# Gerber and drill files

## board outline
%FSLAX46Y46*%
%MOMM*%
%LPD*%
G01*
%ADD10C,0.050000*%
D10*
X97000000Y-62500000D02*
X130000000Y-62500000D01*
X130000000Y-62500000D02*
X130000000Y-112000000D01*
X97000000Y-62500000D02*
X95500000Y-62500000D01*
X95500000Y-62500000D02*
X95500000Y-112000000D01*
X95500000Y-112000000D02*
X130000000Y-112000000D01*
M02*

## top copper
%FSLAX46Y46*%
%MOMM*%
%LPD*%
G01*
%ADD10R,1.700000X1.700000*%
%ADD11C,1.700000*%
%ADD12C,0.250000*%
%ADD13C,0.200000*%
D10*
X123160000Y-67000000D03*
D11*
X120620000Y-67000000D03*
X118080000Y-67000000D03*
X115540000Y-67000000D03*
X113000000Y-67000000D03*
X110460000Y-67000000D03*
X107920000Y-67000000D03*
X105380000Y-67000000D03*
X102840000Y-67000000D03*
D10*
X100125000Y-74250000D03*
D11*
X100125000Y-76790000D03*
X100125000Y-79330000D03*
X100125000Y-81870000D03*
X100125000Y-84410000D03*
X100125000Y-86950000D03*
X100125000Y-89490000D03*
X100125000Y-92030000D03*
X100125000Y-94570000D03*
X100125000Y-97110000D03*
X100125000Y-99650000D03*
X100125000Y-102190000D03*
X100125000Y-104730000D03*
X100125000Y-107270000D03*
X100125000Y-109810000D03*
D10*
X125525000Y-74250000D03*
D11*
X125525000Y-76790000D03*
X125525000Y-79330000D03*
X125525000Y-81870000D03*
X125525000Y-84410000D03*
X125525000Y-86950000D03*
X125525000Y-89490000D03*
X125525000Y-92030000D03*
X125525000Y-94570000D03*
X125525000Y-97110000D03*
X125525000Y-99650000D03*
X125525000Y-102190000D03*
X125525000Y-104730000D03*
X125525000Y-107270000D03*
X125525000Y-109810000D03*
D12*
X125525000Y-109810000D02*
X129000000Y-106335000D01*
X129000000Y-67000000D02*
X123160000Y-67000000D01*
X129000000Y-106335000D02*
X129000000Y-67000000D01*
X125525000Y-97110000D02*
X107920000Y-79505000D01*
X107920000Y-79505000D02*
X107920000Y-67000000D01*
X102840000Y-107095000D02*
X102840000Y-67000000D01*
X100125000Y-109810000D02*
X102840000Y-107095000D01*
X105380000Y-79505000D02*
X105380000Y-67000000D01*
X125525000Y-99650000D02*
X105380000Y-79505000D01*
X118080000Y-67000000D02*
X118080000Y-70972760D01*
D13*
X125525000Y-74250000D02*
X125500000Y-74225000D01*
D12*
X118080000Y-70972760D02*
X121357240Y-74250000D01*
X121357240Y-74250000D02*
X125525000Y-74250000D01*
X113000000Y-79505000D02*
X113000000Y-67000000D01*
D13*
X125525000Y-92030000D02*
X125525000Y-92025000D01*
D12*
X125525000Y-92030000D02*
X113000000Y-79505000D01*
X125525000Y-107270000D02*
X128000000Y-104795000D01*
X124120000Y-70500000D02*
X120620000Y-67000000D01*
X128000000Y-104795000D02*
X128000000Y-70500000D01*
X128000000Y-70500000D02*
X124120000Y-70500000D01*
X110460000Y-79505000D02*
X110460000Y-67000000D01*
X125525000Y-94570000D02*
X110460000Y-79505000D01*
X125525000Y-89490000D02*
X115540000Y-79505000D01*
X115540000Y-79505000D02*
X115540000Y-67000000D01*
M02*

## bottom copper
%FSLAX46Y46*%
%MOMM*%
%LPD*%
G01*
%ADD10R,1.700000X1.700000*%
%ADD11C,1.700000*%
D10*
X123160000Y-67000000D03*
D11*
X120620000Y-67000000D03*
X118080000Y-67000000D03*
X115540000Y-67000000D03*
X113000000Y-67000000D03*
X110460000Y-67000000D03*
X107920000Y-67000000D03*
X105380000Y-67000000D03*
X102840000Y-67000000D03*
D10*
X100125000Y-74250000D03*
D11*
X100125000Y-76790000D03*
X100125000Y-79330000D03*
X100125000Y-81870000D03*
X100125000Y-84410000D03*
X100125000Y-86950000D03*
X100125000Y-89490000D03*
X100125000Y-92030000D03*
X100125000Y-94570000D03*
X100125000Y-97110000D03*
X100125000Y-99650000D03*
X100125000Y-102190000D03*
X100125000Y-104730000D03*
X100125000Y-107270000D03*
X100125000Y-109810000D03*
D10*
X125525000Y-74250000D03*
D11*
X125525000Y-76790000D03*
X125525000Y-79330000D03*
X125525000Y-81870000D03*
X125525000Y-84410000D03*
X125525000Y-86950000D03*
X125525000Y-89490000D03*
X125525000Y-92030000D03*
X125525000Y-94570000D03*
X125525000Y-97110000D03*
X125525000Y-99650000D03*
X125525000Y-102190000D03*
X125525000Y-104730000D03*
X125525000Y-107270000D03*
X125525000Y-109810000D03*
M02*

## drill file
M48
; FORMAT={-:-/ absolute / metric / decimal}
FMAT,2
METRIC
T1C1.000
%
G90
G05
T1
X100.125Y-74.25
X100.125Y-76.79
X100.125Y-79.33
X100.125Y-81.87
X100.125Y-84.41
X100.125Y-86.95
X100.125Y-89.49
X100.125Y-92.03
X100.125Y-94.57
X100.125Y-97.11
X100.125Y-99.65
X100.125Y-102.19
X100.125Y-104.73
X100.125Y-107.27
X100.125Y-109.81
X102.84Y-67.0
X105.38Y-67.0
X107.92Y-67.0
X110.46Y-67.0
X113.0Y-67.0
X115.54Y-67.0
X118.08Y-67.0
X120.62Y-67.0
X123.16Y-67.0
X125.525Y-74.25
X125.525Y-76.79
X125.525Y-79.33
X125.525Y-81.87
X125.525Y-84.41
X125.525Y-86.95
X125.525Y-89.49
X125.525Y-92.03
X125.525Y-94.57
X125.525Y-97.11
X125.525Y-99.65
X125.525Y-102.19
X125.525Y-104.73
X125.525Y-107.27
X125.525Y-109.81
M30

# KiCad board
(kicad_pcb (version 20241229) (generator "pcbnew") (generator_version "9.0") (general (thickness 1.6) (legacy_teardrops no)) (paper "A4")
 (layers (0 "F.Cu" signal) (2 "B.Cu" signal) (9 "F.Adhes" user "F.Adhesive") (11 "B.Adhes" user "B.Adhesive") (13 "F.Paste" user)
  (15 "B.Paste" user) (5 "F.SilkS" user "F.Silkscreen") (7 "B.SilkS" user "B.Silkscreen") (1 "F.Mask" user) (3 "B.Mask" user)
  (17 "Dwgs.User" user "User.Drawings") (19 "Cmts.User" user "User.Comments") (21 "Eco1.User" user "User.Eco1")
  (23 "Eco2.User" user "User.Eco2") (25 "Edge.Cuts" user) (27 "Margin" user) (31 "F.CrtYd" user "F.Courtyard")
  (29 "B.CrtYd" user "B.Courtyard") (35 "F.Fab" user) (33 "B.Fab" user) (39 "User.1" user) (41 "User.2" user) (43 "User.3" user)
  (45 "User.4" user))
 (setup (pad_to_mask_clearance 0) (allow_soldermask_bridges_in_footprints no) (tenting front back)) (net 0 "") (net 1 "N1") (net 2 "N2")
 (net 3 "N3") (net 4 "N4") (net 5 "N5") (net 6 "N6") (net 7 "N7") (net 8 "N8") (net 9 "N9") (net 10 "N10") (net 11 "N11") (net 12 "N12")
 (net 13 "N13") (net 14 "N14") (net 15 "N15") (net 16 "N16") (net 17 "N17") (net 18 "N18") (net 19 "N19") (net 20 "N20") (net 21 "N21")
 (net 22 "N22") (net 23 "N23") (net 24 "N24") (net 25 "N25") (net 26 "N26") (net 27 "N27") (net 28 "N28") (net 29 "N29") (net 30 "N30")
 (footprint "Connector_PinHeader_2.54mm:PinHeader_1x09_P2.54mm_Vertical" (layer "F.Cu") (at 123.16 67 -90)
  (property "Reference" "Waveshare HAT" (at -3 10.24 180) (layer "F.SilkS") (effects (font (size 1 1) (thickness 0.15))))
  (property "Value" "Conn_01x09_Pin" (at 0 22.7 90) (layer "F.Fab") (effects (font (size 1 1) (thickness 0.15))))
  (pad "1" thru_hole rect (at 0 0 270) (size 1.7 1.7) (drill 1) (layers "*.Cu" "*.Mask") (remove_unused_layers no) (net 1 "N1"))
  (pad "2" thru_hole circle (at 0 2.54 270) (size 1.7 1.7) (drill 1) (layers "*.Cu" "*.Mask") (remove_unused_layers no) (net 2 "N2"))
  (pad "3" thru_hole circle (at 0 5.08 270) (size 1.7 1.7) (drill 1) (layers "*.Cu" "*.Mask") (remove_unused_layers no) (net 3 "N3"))
  (pad "4" thru_hole circle (at 0 7.62 270) (size 1.7 1.7) (drill 1) (layers "*.Cu" "*.Mask") (remove_unused_layers no) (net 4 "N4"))
  (pad "5" thru_hole circle (at 0 10.16 270) (size 1.7 1.7) (drill 1) (layers "*.Cu" "*.Mask") (remove_unused_layers no) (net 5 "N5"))
  (pad "6" thru_hole circle (at 0 12.7 270) (size 1.7 1.7) (drill 1) (layers "*.Cu" "*.Mask") (remove_unused_layers no) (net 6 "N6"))
  (pad "7" thru_hole circle (at 0 15.24 270) (size 1.7 1.7) (drill 1) (layers "*.Cu" "*.Mask") (remove_unused_layers no) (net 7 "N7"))
  (pad "8" thru_hole circle (at 0 17.78 270) (size 1.7 1.7) (drill 1) (layers "*.Cu" "*.Mask") (remove_unused_layers no) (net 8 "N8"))
  (pad "9" thru_hole circle (at 0 20.32 270) (size 1.7 1.7) (drill 1) (layers "*.Cu" "*.Mask") (remove_unused_layers no) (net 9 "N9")))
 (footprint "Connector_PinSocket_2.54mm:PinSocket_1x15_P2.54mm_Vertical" (layer "F.Cu") (at 100.125 74.25)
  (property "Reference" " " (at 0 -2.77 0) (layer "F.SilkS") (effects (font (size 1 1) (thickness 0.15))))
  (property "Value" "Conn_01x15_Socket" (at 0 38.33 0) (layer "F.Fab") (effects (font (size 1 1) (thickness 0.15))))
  (pad "1" thru_hole rect (at 0 0) (size 1.7 1.7) (drill 1) (layers "*.Cu" "*.Mask") (remove_unused_layers no) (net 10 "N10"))
  (pad "2" thru_hole circle (at 0 2.54) (size 1.7 1.7) (drill 1) (layers "*.Cu" "*.Mask") (remove_unused_layers no) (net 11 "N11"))
  (pad "3" thru_hole circle (at 0 5.08) (size 1.7 1.7) (drill 1) (layers "*.Cu" "*.Mask") (remove_unused_layers no) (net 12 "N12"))
  (pad "4" thru_hole circle (at 0 7.62) (size 1.7 1.7) (drill 1) (layers "*.Cu" "*.Mask") (remove_unused_layers no) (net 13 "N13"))
  (pad "5" thru_hole circle (at 0 10.16) (size 1.7 1.7) (drill 1) (layers "*.Cu" "*.Mask") (remove_unused_layers no) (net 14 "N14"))
  (pad "6" thru_hole circle (at 0 12.7) (size 1.7 1.7) (drill 1) (layers "*.Cu" "*.Mask") (remove_unused_layers no) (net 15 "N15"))
  (pad "7" thru_hole circle (at 0 15.24) (size 1.7 1.7) (drill 1) (layers "*.Cu" "*.Mask") (remove_unused_layers no) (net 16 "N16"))
  (pad "8" thru_hole circle (at 0 17.78) (size 1.7 1.7) (drill 1) (layers "*.Cu" "*.Mask") (remove_unused_layers no) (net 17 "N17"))
  (pad "9" thru_hole circle (at 0 20.32) (size 1.7 1.7) (drill 1) (layers "*.Cu" "*.Mask") (remove_unused_layers no) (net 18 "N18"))
  (pad "10" thru_hole circle (at 0 22.86) (size 1.7 1.7) (drill 1) (layers "*.Cu" "*.Mask") (remove_unused_layers no) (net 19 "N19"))
  (pad "11" thru_hole circle (at 0 25.4) (size 1.7 1.7) (drill 1) (layers "*.Cu" "*.Mask") (remove_unused_layers no) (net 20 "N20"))
  (pad "12" thru_hole circle (at 0 27.94) (size 1.7 1.7) (drill 1) (layers "*.Cu" "*.Mask") (remove_unused_layers no) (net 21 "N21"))
  (pad "13" thru_hole circle (at 0 30.48) (size 1.7 1.7) (drill 1) (layers "*.Cu" "*.Mask") (remove_unused_layers no) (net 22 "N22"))
  (pad "14" thru_hole circle (at 0 33.02) (size 1.7 1.7) (drill 1) (layers "*.Cu" "*.Mask") (remove_unused_layers no) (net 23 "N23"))
  (pad "15" thru_hole circle (at 0 35.56) (size 1.7 1.7) (drill 1) (layers "*.Cu" "*.Mask") (remove_unused_layers no) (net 9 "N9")))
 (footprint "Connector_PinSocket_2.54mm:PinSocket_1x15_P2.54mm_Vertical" (layer "F.Cu") (at 125.525 74.25)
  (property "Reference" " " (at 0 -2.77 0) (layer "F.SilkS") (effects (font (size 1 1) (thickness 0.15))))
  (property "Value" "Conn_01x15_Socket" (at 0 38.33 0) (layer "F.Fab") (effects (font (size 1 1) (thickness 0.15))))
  (pad "1" thru_hole rect (at 0 0) (size 1.7 1.7) (drill 1) (layers "*.Cu" "*.Mask") (remove_unused_layers no) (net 3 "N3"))
  (pad "2" thru_hole circle (at 0 2.54) (size 1.7 1.7) (drill 1) (layers "*.Cu" "*.Mask") (remove_unused_layers no) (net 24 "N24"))
  (pad "3" thru_hole circle (at 0 5.08) (size 1.7 1.7) (drill 1) (layers "*.Cu" "*.Mask") (remove_unused_layers no) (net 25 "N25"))
  (pad "4" thru_hole circle (at 0 7.62) (size 1.7 1.7) (drill 1) (layers "*.Cu" "*.Mask") (remove_unused_layers no) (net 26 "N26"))
  (pad "5" thru_hole circle (at 0 10.16) (size 1.7 1.7) (drill 1) (layers "*.Cu" "*.Mask") (remove_unused_layers no) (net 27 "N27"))
  (pad "6" thru_hole circle (at 0 12.7) (size 1.7 1.7) (drill 1) (layers "*.Cu" "*.Mask") (remove_unused_layers no) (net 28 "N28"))
  (pad "7" thru_hole circle (at 0 15.24) (size 1.7 1.7) (drill 1) (layers "*.Cu" "*.Mask") (remove_unused_layers no) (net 4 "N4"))
  (pad "8" thru_hole circle (at 0 17.78) (size 1.7 1.7) (drill 1) (layers "*.Cu" "*.Mask") (remove_unused_layers no) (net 5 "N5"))
  (pad "9" thru_hole circle (at 0 20.32) (size 1.7 1.7) (drill 1) (layers "*.Cu" "*.Mask") (remove_unused_layers no) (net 6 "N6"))
  (pad "10" thru_hole circle (at 0 22.86) (size 1.7 1.7) (drill 1) (layers "*.Cu" "*.Mask") (remove_unused_layers no) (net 7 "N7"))
  (pad "11" thru_hole circle (at 0 25.4) (size 1.7 1.7) (drill 1) (layers "*.Cu" "*.Mask") (remove_unused_layers no) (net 8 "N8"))
  (pad "12" thru_hole circle (at 0 27.94) (size 1.7 1.7) (drill 1) (layers "*.Cu" "*.Mask") (remove_unused_layers no) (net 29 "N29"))
  (pad "13" thru_hole circle (at 0 30.48) (size 1.7 1.7) (drill 1) (layers "*.Cu" "*.Mask") (remove_unused_layers no) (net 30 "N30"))
  (pad "14" thru_hole circle (at 0 33.02) (size 1.7 1.7) (drill 1) (layers "*.Cu" "*.Mask") (remove_unused_layers no) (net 2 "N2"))
  (pad "15" thru_hole circle (at 0 35.56) (size 1.7 1.7) (drill 1) (layers "*.Cu" "*.Mask") (remove_unused_layers no) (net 1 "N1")))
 (gr_line (start 97 62.5) (end 130 62.5) (stroke (width 0.05) (type default)) (layer "Edge.Cuts"))
 (gr_line (start 130 62.5) (end 130 112) (stroke (width 0.05) (type default)) (layer "Edge.Cuts"))
 (gr_line (start 97 62.5) (end 95.5 62.5) (stroke (width 0.05) (type default)) (layer "Edge.Cuts"))
 (gr_line (start 95.5 62.5) (end 95.5 112) (stroke (width 0.05) (type default)) (layer "Edge.Cuts"))
 (gr_line (start 95.5 112) (end 130 112) (stroke (width 0.05) (type default)) (layer "Edge.Cuts"))
 (segment (start 125.525 109.81) (end 129 106.335) (width 0.25) (layer "F.Cu") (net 1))
 (segment (start 129 67) (end 123.16 67) (width 0.25) (layer "F.Cu") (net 1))
 (segment (start 129 106.335) (end 129 67) (width 0.25) (layer "F.Cu") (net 1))
 (segment (start 125.525 97.11) (end 107.92 79.505) (width 0.25) (layer "F.Cu") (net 7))
 (segment (start 107.92 79.505) (end 107.92 67) (width 0.25) (layer "F.Cu") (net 7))
 (segment (start 102.84 107.095) (end 102.84 67) (width 0.25) (layer "F.Cu") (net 9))
 (segment (start 100.125 109.81) (end 102.84 107.095) (width 0.25) (layer "F.Cu") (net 9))
 (segment (start 105.38 79.505) (end 105.38 67) (width 0.25) (layer "F.Cu") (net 8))
 (segment (start 125.525 99.65) (end 105.38 79.505) (width 0.25) (layer "F.Cu") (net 8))
 (segment (start 118.08 67) (end 118.08 70.97276) (width 0.25) (layer "F.Cu") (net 3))
 (segment (start 125.525 74.25) (end 125.5 74.225) (width 0.2) (layer "F.Cu") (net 3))
 (segment (start 118.08 70.97276) (end 121.35724 74.25) (width 0.25) (layer "F.Cu") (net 3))
 (segment (start 121.35724 74.25) (end 125.525 74.25) (width 0.25) (layer "F.Cu") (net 3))
 (segment (start 113 79.505) (end 113 67) (width 0.25) (layer "F.Cu") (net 5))
 (segment (start 125.525 92.03) (end 125.525 92.025) (width 0.2) (layer "F.Cu") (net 5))
 (segment (start 125.525 92.03) (end 113 79.505) (width 0.25) (layer "F.Cu") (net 5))
 (segment (start 125.525 107.27) (end 128 104.795) (width 0.25) (layer "F.Cu") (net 2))
 (segment (start 124.12 70.5) (end 120.62 67) (width 0.25) (layer "F.Cu") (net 2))
 (segment (start 128 104.795) (end 128 70.5) (width 0.25) (layer "F.Cu") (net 2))
 (segment (start 128 70.5) (end 124.12 70.5) (width 0.25) (layer "F.Cu") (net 2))
 (segment (start 110.46 79.505) (end 110.46 67) (width 0.25) (layer "F.Cu") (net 6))
 (segment (start 125.525 94.57) (end 110.46 79.505) (width 0.25) (layer "F.Cu") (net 6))
 (segment (start 125.525 89.49) (end 115.54 79.505) (width 0.25) (layer "F.Cu") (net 4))
 (segment (start 115.54 79.505) (end 115.54 67) (width 0.25) (layer "F.Cu") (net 4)))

